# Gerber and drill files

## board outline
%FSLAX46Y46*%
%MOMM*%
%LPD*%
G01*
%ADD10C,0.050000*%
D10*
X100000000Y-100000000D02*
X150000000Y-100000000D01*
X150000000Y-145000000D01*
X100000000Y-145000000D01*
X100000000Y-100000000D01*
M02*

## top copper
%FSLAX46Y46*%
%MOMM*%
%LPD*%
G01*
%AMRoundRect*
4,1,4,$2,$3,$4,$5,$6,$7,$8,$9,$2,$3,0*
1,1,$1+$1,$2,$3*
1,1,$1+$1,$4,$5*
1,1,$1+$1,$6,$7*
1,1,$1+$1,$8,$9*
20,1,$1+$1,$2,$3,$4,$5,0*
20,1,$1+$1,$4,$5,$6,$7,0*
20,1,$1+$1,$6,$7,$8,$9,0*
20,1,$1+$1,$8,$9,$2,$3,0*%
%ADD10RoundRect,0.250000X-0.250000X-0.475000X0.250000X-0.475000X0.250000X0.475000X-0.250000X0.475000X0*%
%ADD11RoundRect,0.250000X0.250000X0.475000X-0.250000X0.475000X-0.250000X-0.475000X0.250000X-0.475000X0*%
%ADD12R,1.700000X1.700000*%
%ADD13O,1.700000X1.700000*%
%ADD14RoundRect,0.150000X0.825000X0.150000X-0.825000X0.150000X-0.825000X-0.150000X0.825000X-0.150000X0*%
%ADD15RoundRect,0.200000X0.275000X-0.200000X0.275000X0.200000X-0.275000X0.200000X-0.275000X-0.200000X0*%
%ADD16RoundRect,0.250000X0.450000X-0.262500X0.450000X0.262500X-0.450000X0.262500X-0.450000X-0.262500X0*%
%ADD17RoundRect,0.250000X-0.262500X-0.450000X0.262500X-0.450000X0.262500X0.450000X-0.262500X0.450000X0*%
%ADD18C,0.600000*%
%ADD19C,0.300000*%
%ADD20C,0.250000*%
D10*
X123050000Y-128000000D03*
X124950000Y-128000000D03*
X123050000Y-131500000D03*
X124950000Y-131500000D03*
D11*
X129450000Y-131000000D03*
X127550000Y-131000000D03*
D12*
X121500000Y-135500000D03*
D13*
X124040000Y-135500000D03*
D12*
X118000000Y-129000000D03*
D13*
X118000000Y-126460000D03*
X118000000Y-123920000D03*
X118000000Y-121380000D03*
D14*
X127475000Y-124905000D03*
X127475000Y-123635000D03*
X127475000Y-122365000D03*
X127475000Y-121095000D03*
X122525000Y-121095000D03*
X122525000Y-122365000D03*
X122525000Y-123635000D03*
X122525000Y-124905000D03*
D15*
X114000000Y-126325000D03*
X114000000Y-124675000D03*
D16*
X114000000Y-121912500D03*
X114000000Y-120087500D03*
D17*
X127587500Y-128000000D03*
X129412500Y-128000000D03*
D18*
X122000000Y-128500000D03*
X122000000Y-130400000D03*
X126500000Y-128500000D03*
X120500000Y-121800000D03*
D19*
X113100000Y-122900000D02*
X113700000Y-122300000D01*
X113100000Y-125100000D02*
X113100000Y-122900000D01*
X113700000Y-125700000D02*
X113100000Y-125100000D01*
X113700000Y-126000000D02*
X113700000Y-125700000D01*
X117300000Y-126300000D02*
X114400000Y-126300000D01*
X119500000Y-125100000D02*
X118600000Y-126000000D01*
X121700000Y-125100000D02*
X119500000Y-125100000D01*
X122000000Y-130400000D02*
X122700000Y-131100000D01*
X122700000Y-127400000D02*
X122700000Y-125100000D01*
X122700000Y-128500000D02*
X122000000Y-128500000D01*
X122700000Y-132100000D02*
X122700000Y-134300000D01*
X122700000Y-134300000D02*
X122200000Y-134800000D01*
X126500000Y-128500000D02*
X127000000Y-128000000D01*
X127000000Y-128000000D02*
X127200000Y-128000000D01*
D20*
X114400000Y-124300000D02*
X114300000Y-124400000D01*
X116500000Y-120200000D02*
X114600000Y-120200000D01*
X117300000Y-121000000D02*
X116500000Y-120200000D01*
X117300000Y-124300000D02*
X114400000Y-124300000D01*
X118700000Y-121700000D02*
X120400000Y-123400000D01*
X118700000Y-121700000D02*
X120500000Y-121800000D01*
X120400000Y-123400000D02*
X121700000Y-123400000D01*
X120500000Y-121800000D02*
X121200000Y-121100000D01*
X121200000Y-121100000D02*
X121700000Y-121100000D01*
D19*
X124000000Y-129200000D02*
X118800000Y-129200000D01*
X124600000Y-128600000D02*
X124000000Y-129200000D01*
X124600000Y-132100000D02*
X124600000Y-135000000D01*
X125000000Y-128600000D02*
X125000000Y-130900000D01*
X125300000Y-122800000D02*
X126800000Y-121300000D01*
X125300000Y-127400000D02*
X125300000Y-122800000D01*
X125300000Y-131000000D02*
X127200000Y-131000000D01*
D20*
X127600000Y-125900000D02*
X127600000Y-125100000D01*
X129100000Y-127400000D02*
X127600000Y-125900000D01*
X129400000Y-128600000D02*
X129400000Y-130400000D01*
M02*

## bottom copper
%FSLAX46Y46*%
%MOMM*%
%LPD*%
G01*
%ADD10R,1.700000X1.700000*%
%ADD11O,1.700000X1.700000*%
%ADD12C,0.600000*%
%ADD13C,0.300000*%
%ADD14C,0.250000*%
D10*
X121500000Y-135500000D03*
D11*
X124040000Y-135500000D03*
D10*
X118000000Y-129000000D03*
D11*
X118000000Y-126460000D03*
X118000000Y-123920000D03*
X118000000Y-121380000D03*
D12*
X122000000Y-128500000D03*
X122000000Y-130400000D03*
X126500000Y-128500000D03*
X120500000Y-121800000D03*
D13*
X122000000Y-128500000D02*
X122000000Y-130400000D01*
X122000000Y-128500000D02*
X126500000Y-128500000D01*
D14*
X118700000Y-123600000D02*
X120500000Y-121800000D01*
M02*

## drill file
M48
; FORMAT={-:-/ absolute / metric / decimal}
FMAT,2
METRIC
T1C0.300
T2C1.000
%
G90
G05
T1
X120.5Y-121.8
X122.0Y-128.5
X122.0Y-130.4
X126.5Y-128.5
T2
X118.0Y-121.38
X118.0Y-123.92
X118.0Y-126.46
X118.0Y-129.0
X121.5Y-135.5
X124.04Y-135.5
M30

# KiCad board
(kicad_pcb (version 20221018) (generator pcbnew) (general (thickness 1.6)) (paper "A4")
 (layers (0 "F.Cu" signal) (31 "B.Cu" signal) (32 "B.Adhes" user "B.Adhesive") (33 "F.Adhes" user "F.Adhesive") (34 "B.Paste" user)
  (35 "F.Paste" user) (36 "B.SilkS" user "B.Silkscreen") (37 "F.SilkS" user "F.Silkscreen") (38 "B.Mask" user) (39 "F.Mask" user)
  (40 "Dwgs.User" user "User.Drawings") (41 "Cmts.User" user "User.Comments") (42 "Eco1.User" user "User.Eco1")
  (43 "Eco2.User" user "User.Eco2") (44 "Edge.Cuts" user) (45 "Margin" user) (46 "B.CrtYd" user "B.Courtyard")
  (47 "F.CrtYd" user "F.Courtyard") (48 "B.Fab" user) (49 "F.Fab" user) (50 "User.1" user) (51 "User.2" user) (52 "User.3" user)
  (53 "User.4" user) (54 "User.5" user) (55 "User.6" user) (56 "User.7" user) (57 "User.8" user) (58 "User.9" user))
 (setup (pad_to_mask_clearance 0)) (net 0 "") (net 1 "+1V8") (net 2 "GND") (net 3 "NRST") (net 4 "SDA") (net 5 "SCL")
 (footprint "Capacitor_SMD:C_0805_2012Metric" (layer "F.Cu") (at 124 128)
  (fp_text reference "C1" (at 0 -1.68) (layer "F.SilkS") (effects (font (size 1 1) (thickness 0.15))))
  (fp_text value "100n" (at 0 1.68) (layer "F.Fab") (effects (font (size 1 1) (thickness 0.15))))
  (pad "1" smd roundrect (at -0.95 0) (size 1 1.45) (layers "F.Cu" "F.Paste" "F.Mask") (roundrect_rratio 0.25) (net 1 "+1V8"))
  (pad "2" smd roundrect (at 0.95 0) (size 1 1.45) (layers "F.Cu" "F.Paste" "F.Mask") (roundrect_rratio 0.25) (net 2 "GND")))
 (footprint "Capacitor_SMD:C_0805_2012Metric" (layer "F.Cu") (at 124 131.5)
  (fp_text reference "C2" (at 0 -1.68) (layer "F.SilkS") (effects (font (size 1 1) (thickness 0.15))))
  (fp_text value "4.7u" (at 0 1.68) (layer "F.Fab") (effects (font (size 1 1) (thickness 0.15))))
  (pad "1" smd roundrect (at -0.95 0) (size 1 1.45) (layers "F.Cu" "F.Paste" "F.Mask") (roundrect_rratio 0.25) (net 1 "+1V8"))
  (pad "2" smd roundrect (at 0.95 0) (size 1 1.45) (layers "F.Cu" "F.Paste" "F.Mask") (roundrect_rratio 0.25) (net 2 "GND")))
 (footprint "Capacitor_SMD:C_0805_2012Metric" (layer "F.Cu") (at 128.5 131 180)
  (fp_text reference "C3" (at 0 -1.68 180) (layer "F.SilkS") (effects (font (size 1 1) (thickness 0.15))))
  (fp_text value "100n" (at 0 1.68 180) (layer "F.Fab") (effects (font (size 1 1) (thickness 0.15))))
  (pad "1" smd roundrect (at -0.95 0 180) (size 1 1.45) (layers "F.Cu" "F.Paste" "F.Mask") (roundrect_rratio 0.25) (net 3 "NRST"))
  (pad "2" smd roundrect (at 0.95 0 180) (size 1 1.45) (layers "F.Cu" "F.Paste" "F.Mask") (roundrect_rratio 0.25) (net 2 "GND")))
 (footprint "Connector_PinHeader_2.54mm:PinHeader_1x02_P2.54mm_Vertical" (layer "F.Cu") (at 121.5 135.5 90)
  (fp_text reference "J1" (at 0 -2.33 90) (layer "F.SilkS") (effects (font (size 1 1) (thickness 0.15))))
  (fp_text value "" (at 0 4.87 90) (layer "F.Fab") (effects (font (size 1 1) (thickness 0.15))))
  (pad "1" thru_hole rect (at 0 0 90) (size 1.7 1.7) (drill 1) (layers "*.Cu" "*.Mask") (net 1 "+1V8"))
  (pad "2" thru_hole oval (at 0 2.54 90) (size 1.7 1.7) (drill 1) (layers "*.Cu" "*.Mask") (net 2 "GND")))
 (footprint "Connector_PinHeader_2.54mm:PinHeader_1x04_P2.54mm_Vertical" (layer "F.Cu") (at 118 129 180)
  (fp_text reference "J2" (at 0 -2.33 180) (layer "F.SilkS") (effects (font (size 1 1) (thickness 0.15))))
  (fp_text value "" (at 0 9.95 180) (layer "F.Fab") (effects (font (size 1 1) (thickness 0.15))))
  (pad "1" thru_hole rect (at 0 0 180) (size 1.7 1.7) (drill 1) (layers "*.Cu" "*.Mask") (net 2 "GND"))
  (pad "2" thru_hole oval (at 0 2.54 180) (size 1.7 1.7) (drill 1) (layers "*.Cu" "*.Mask") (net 1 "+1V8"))
  (pad "3" thru_hole oval (at 0 5.08 180) (size 1.7 1.7) (drill 1) (layers "*.Cu" "*.Mask") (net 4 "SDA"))
  (pad "4" thru_hole oval (at 0 7.62 180) (size 1.7 1.7) (drill 1) (layers "*.Cu" "*.Mask") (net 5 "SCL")))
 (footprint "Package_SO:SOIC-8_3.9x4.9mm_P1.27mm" (layer "F.Cu") (at 125 123 180)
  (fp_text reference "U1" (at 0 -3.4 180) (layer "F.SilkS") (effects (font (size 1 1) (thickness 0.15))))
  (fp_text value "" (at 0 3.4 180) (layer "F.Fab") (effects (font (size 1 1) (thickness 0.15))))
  (pad "1" smd roundrect (at -2.475 -1.905 180) (size 1.95 0.6) (layers "F.Cu" "F.Paste" "F.Mask") (roundrect_rratio 0.25) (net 3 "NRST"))
  (pad "2" smd roundrect (at -2.475 -0.635 180) (size 1.95 0.6) (layers "F.Cu" "F.Paste" "F.Mask") (roundrect_rratio 0.25))
  (pad "3" smd roundrect (at -2.475 0.635 180) (size 1.95 0.6) (layers "F.Cu" "F.Paste" "F.Mask") (roundrect_rratio 0.25))
  (pad "4" smd roundrect (at -2.475 1.905 180) (size 1.95 0.6) (layers "F.Cu" "F.Paste" "F.Mask") (roundrect_rratio 0.25) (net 2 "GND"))
  (pad "5" smd roundrect (at 2.475 1.905 180) (size 1.95 0.6) (layers "F.Cu" "F.Paste" "F.Mask") (roundrect_rratio 0.25) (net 4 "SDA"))
  (pad "6" smd roundrect (at 2.475 0.635 180) (size 1.95 0.6) (layers "F.Cu" "F.Paste" "F.Mask") (roundrect_rratio 0.25))
  (pad "7" smd roundrect (at 2.475 -0.635 180) (size 1.95 0.6) (layers "F.Cu" "F.Paste" "F.Mask") (roundrect_rratio 0.25) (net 5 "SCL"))
  (pad "8" smd roundrect (at 2.475 -1.905 180) (size 1.95 0.6) (layers "F.Cu" "F.Paste" "F.Mask") (roundrect_rratio 0.25) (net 1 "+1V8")))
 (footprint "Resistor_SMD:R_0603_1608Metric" (layer "F.Cu") (at 114 125.5 90)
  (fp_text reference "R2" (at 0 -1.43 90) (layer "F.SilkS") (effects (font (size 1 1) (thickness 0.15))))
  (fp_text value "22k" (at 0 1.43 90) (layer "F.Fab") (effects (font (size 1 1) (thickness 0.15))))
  (pad "1" smd roundrect (at -0.825 0 90) (size 0.8 0.95) (layers "F.Cu" "F.Paste" "F.Mask") (roundrect_rratio 0.25) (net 1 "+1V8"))
  (pad "2" smd roundrect (at 0.825 0 90) (size 0.8 0.95) (layers "F.Cu" "F.Paste" "F.Mask") (roundrect_rratio 0.25) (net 4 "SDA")))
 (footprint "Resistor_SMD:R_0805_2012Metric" (layer "F.Cu") (at 114 121 90)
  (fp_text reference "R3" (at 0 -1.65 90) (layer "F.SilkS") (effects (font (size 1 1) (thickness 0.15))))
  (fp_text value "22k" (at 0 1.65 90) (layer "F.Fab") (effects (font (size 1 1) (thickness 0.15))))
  (pad "1" smd roundrect (at -0.9125 0 90) (size 1.025 1.4) (layers "F.Cu" "F.Paste" "F.Mask") (roundrect_rratio 0.243902) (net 1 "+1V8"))
  (pad "2" smd roundrect (at 0.9125 0 90) (size 1.025 1.4) (layers "F.Cu" "F.Paste" "F.Mask") (roundrect_rratio 0.243902) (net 5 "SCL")))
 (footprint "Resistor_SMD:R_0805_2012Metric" (layer "F.Cu") (at 128.5 128)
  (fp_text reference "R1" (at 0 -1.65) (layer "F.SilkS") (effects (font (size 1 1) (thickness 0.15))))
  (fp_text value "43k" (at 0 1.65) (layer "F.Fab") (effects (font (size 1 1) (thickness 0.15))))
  (pad "1" smd roundrect (at -0.9125 0) (size 1.025 1.4) (layers "F.Cu" "F.Paste" "F.Mask") (roundrect_rratio 0.243902) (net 1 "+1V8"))
  (pad "2" smd roundrect (at 0.9125 0) (size 1.025 1.4) (layers "F.Cu" "F.Paste" "F.Mask") (roundrect_rratio 0.243902) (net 3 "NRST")))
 (gr_rect (start 100 100) (end 150 145) (stroke (width 0.05) (type default)) (fill none) (layer "Edge.Cuts"))
 (segment (start 113.1 122.9) (end 113.7 122.3) (width 0.3) (layer "F.Cu") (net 1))
 (segment (start 113.1 125.1) (end 113.1 122.9) (width 0.3) (layer "F.Cu") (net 1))
 (segment (start 113.7 125.7) (end 113.1 125.1) (width 0.3) (layer "F.Cu") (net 1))
 (segment (start 113.7 126) (end 113.7 125.7) (width 0.3) (layer "F.Cu") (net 1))
 (segment (start 117.3 126.3) (end 114.4 126.3) (width 0.3) (layer "F.Cu") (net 1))
 (segment (start 119.5 125.1) (end 118.6 126) (width 0.3) (layer "F.Cu") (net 1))
 (segment (start 121.7 125.1) (end 119.5 125.1) (width 0.3) (layer "F.Cu") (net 1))
 (segment (start 122 130.4) (end 122.7 131.1) (width 0.3) (layer "F.Cu") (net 1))
 (segment (start 122.7 127.4) (end 122.7 125.1) (width 0.3) (layer "F.Cu") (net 1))
 (segment (start 122.7 128.5) (end 122 128.5) (width 0.3) (layer "F.Cu") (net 1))
 (segment (start 122.7 132.1) (end 122.7 134.3) (width 0.3) (layer "F.Cu") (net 1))
 (segment (start 122.7 134.3) (end 122.2 134.8) (width 0.3) (layer "F.Cu") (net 1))
 (segment (start 126.5 128.5) (end 127 128) (width 0.3) (layer "F.Cu") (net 1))
 (segment (start 127 128) (end 127.2 128) (width 0.3) (layer "F.Cu") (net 1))
 (via (at 122 128.5) (size 0.6) (drill 0.3) (layers "F.Cu" "B.Cu") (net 1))
 (via (at 122 130.4) (size 0.6) (drill 0.3) (layers "F.Cu" "B.Cu") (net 1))
 (via (at 126.5 128.5) (size 0.6) (drill 0.3) (layers "F.Cu" "B.Cu") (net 1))
 (segment (start 114.4 124.3) (end 114.3 124.4) (width 0.25) (layer "F.Cu") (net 4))
 (segment (start 116.5 120.2) (end 114.6 120.2) (width 0.25) (layer "F.Cu") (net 5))
 (segment (start 117.3 121) (end 116.5 120.2) (width 0.25) (layer "F.Cu") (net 5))
 (segment (start 117.3 124.3) (end 114.4 124.3) (width 0.25) (layer "F.Cu") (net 4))
 (segment (start 118.7 121.7) (end 120.4 123.4) (width 0.25) (layer "F.Cu") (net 5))
 (segment (start 118.7 121.7) (end 120.5 121.8) (width 0.25) (layer "F.Cu") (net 5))
 (segment (start 120.4 123.4) (end 121.7 123.4) (width 0.25) (layer "F.Cu") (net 5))
 (segment (start 120.5 121.8) (end 121.2 121.1) (width 0.25) (layer "F.Cu") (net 4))
 (segment (start 121.2 121.1) (end 121.7 121.1) (width 0.25) (layer "F.Cu") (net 4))
 (segment (start 122 128.5) (end 122 130.4) (width 0.3) (layer "B.Cu") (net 1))
 (segment (start 122 128.5) (end 126.5 128.5) (width 0.3) (layer "B.Cu") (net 1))
 (segment (start 124 129.2) (end 118.8 129.2) (width 0.3) (layer "F.Cu") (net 2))
 (segment (start 124.6 128.6) (end 124 129.2) (width 0.3) (layer "F.Cu") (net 2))
 (segment (start 124.6 132.1) (end 124.6 135) (width 0.3) (layer "F.Cu") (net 2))
 (segment (start 125 128.6) (end 125 130.9) (width 0.3) (layer "F.Cu") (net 2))
 (segment (start 125.3 122.8) (end 126.8 121.3) (width 0.3) (layer "F.Cu") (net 2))
 (segment (start 125.3 127.4) (end 125.3 122.8) (width 0.3) (layer "F.Cu") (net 2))
 (segment (start 125.3 131) (end 127.2 131) (width 0.3) (layer "F.Cu") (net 2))
 (segment (start 127.6 125.9) (end 127.6 125.1) (width 0.25) (layer "F.Cu") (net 3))
 (segment (start 129.1 127.4) (end 127.6 125.9) (width 0.25) (layer "F.Cu") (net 3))
 (segment (start 129.4 128.6) (end 129.4 130.4) (width 0.25) (layer "F.Cu") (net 3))
 (via (at 120.5 121.8) (size 0.6) (drill 0.3) (layers "F.Cu" "B.Cu") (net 4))
 (segment (start 118.7 123.6) (end 120.5 121.8) (width 0.25) (layer "B.Cu") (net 4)))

